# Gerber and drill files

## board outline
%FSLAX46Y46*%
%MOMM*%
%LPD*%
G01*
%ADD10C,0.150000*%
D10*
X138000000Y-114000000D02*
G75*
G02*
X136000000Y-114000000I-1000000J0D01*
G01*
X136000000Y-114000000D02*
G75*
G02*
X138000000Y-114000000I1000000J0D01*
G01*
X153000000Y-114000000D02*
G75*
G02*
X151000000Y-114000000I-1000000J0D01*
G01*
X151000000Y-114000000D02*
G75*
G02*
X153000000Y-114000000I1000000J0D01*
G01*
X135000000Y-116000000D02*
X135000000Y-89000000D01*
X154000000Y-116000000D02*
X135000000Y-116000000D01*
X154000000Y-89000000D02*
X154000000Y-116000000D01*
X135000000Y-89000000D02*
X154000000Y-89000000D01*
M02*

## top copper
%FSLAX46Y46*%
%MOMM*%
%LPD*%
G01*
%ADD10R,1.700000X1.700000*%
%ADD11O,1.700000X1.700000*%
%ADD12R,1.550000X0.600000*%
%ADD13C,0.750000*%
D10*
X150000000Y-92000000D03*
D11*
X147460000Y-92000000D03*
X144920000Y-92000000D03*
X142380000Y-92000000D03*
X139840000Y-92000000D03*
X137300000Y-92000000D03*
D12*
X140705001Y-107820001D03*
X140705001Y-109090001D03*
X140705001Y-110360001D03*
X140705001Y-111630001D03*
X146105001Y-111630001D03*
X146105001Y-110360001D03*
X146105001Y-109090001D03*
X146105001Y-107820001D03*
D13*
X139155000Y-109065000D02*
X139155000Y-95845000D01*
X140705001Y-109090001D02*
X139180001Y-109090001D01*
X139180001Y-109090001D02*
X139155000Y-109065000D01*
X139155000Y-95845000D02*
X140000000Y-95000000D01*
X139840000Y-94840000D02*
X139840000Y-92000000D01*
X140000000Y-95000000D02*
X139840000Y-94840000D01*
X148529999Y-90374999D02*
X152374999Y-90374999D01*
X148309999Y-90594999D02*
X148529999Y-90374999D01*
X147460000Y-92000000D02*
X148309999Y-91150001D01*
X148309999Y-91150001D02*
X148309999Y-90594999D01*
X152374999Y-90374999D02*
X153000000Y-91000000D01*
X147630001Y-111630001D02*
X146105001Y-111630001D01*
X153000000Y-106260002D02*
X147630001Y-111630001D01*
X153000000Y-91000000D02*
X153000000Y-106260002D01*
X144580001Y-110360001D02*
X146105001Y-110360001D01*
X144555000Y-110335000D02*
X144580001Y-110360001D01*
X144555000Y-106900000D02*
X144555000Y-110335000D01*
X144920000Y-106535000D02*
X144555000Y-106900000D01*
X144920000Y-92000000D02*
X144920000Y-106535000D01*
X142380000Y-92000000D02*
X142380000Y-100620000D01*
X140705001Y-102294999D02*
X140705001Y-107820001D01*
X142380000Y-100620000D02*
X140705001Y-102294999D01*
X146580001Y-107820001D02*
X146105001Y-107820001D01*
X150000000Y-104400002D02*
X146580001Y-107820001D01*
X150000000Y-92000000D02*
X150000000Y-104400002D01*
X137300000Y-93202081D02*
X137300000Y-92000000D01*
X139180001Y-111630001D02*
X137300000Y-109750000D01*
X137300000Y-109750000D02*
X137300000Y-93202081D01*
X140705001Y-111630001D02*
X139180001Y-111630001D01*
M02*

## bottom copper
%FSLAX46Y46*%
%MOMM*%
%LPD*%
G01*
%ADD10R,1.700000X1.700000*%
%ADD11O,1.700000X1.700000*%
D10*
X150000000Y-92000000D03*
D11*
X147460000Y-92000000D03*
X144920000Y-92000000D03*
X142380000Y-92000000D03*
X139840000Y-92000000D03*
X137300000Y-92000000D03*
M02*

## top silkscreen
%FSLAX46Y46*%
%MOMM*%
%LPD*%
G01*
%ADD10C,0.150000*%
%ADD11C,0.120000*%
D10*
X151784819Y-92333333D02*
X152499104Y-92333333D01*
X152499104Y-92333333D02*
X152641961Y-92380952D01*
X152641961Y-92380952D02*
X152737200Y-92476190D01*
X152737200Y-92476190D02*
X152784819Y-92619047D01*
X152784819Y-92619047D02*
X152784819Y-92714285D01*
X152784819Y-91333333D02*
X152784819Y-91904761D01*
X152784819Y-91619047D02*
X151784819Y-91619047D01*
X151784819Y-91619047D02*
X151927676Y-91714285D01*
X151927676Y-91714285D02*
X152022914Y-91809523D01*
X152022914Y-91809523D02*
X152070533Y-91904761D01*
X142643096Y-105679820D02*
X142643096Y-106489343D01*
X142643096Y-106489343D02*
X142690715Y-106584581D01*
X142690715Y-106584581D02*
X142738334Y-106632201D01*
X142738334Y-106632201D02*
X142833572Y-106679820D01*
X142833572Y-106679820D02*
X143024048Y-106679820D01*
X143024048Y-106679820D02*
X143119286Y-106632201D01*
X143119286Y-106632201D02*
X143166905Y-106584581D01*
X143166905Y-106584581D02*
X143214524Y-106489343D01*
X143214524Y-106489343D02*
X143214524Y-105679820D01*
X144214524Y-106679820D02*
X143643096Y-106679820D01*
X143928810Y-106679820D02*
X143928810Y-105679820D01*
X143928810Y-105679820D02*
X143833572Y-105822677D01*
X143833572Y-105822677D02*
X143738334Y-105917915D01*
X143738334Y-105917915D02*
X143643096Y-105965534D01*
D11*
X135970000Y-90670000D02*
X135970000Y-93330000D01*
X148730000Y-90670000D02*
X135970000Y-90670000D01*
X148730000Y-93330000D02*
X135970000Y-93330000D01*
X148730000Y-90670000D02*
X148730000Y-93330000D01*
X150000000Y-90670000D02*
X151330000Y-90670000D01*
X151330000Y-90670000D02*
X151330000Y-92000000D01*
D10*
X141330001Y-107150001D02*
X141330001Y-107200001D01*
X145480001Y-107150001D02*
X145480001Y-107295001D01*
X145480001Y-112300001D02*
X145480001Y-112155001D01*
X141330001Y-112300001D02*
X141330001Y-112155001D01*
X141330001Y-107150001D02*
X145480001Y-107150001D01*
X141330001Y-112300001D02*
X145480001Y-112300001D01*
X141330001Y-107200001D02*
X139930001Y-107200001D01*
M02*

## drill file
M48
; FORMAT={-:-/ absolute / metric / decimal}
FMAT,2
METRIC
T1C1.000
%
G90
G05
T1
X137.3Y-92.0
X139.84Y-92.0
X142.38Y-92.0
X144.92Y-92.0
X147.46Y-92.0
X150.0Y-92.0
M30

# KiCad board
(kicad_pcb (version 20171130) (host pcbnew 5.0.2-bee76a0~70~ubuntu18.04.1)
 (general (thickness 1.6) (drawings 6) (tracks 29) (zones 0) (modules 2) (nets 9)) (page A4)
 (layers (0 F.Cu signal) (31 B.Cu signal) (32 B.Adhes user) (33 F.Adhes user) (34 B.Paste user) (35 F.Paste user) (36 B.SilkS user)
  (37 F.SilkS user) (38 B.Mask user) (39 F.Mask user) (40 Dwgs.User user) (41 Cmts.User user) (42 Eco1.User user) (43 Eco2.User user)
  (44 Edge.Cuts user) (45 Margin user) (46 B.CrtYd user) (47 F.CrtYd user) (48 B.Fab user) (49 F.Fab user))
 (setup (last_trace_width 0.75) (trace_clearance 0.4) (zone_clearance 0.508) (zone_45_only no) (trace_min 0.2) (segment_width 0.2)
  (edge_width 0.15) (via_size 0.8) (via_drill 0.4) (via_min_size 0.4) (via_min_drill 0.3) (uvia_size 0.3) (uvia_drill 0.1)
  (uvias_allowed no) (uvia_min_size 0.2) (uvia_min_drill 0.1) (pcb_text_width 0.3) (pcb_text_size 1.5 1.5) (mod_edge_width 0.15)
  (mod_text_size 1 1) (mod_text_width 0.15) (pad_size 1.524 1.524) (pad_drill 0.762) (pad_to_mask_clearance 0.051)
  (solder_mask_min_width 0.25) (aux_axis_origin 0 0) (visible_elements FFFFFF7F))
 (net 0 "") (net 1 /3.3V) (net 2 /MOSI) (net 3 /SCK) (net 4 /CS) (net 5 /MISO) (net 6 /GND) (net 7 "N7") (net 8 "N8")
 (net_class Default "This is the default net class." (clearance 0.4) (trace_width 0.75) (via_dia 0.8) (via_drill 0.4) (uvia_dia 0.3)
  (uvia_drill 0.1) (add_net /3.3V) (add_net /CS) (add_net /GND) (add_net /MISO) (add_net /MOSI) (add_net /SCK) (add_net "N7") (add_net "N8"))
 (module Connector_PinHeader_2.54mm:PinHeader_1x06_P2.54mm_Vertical (layer F.Cu) (at 150 92 270)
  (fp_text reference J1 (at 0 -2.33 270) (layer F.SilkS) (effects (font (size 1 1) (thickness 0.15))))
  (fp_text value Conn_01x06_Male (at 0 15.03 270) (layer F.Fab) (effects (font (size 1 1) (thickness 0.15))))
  (fp_line (start -1.33 14.03) (end 1.33 14.03) (layer F.SilkS) (width 0.12))
  (fp_line (start -1.33 1.27) (end -1.33 14.03) (layer F.SilkS) (width 0.12))
  (fp_line (start 1.33 1.27) (end 1.33 14.03) (layer F.SilkS) (width 0.12))
  (fp_line (start -1.33 1.27) (end 1.33 1.27) (layer F.SilkS) (width 0.12))
  (fp_line (start -1.33 0) (end -1.33 -1.33) (layer F.SilkS) (width 0.12))
  (fp_line (start -1.33 -1.33) (end 0 -1.33) (layer F.SilkS) (width 0.12))
  (pad 1 thru_hole rect (at 0 0 270) (size 1.7 1.7) (drill 1) (layers *.Cu *.Mask) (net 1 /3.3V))
  (pad 2 thru_hole oval (at 0 2.54 270) (size 1.7 1.7) (drill 1) (layers *.Cu *.Mask) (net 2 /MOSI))
  (pad 3 thru_hole oval (at 0 5.08 270) (size 1.7 1.7) (drill 1) (layers *.Cu *.Mask) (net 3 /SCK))
  (pad 4 thru_hole oval (at 0 7.62 270) (size 1.7 1.7) (drill 1) (layers *.Cu *.Mask) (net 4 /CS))
  (pad 5 thru_hole oval (at 0 10.16 270) (size 1.7 1.7) (drill 1) (layers *.Cu *.Mask) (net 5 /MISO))
  (pad 6 thru_hole oval (at 0 12.7 270) (size 1.7 1.7) (drill 1) (layers *.Cu *.Mask) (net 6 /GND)))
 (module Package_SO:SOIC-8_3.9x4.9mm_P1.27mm (layer F.Cu) (at 143.405001 109.725001)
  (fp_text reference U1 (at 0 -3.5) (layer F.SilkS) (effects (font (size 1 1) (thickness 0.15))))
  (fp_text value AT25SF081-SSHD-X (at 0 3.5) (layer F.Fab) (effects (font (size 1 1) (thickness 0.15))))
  (fp_line (start -2.075 -2.575) (end -2.075 -2.525) (layer F.SilkS) (width 0.15))
  (fp_line (start 2.075 -2.575) (end 2.075 -2.43) (layer F.SilkS) (width 0.15))
  (fp_line (start 2.075 2.575) (end 2.075 2.43) (layer F.SilkS) (width 0.15))
  (fp_line (start -2.075 2.575) (end -2.075 2.43) (layer F.SilkS) (width 0.15))
  (fp_line (start -2.075 -2.575) (end 2.075 -2.575) (layer F.SilkS) (width 0.15))
  (fp_line (start -2.075 2.575) (end 2.075 2.575) (layer F.SilkS) (width 0.15))
  (fp_line (start -2.075 -2.525) (end -3.475 -2.525) (layer F.SilkS) (width 0.15))
  (pad 1 smd rect (at -2.7 -1.905) (size 1.55 0.6) (layers F.Cu F.Paste F.Mask) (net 4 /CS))
  (pad 2 smd rect (at -2.7 -0.635) (size 1.55 0.6) (layers F.Cu F.Paste F.Mask) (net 5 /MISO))
  (pad 3 smd rect (at -2.7 0.635) (size 1.55 0.6) (layers F.Cu F.Paste F.Mask) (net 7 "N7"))
  (pad 4 smd rect (at -2.7 1.905) (size 1.55 0.6) (layers F.Cu F.Paste F.Mask) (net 6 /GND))
  (pad 5 smd rect (at 2.7 1.905) (size 1.55 0.6) (layers F.Cu F.Paste F.Mask) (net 2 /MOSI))
  (pad 6 smd rect (at 2.7 0.635) (size 1.55 0.6) (layers F.Cu F.Paste F.Mask) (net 3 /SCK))
  (pad 7 smd rect (at 2.7 -0.635) (size 1.55 0.6) (layers F.Cu F.Paste F.Mask) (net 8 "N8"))
  (pad 8 smd rect (at 2.7 -1.905) (size 1.55 0.6) (layers F.Cu F.Paste F.Mask) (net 1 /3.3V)))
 (gr_circle (center 137 114) (end 138 114) (layer Edge.Cuts) (width 0.15))
 (gr_circle (center 152 114) (end 153 114) (layer Edge.Cuts) (width 0.15))
 (gr_line (start 135 116) (end 135 89) (layer Edge.Cuts) (width 0.15))
 (gr_line (start 154 116) (end 135 116) (layer Edge.Cuts) (width 0.15))
 (gr_line (start 154 89) (end 154 116) (layer Edge.Cuts) (width 0.15))
 (gr_line (start 135 89) (end 154 89) (layer Edge.Cuts) (width 0.15))
 (segment (start 139.155 109.065) (end 139.155 95.845) (width 0.75) (layer F.Cu) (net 5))
 (segment (start 140.705001 109.090001) (end 139.180001 109.090001) (width 0.75) (layer F.Cu) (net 5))
 (segment (start 139.180001 109.090001) (end 139.155 109.065) (width 0.75) (layer F.Cu) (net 5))
 (segment (start 139.155 95.845) (end 140 95) (width 0.75) (layer F.Cu) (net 5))
 (segment (start 139.84 94.84) (end 139.84 92) (width 0.75) (layer F.Cu) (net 5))
 (segment (start 140 95) (end 139.84 94.84) (width 0.75) (layer F.Cu) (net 5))
 (segment (start 148.529999 90.374999) (end 152.374999 90.374999) (width 0.75) (layer F.Cu) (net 2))
 (segment (start 148.309999 90.594999) (end 148.529999 90.374999) (width 0.75) (layer F.Cu) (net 2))
 (segment (start 147.46 92) (end 148.309999 91.150001) (width 0.75) (layer F.Cu) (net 2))
 (segment (start 148.309999 91.150001) (end 148.309999 90.594999) (width 0.75) (layer F.Cu) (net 2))
 (segment (start 152.374999 90.374999) (end 153 91) (width 0.75) (layer F.Cu) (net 2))
 (segment (start 147.630001 111.630001) (end 146.105001 111.630001) (width 0.75) (layer F.Cu) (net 2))
 (segment (start 153 106.260002) (end 147.630001 111.630001) (width 0.75) (layer F.Cu) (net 2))
 (segment (start 153 91) (end 153 106.260002) (width 0.75) (layer F.Cu) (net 2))
 (segment (start 144.580001 110.360001) (end 146.105001 110.360001) (width 0.75) (layer F.Cu) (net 3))
 (segment (start 144.555 110.335) (end 144.580001 110.360001) (width 0.75) (layer F.Cu) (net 3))
 (segment (start 144.555 106.9) (end 144.555 110.335) (width 0.75) (layer F.Cu) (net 3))
 (segment (start 144.92 106.535) (end 144.555 106.9) (width 0.75) (layer F.Cu) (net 3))
 (segment (start 144.92 92) (end 144.92 106.535) (width 0.75) (layer F.Cu) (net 3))
 (segment (start 142.38 92) (end 142.38 100.62) (width 0.75) (layer F.Cu) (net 4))
 (segment (start 140.705001 102.294999) (end 140.705001 107.820001) (width 0.75) (layer F.Cu) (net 4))
 (segment (start 142.38 100.62) (end 140.705001 102.294999) (width 0.75) (layer F.Cu) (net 4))
 (segment (start 146.580001 107.820001) (end 146.105001 107.820001) (width 0.75) (layer F.Cu) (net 1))
 (segment (start 150 104.400002) (end 146.580001 107.820001) (width 0.75) (layer F.Cu) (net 1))
 (segment (start 150 92) (end 150 104.400002) (width 0.75) (layer F.Cu) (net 1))
 (segment (start 137.3 93.202081) (end 137.3 92) (width 0.75) (layer F.Cu) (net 6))
 (segment (start 139.180001 111.630001) (end 137.3 109.75) (width 0.75) (layer F.Cu) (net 6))
 (segment (start 137.3 109.75) (end 137.3 93.202081) (width 0.75) (layer F.Cu) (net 6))
 (segment (start 140.705001 111.630001) (end 139.180001 111.630001) (width 0.75) (layer F.Cu) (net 6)))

